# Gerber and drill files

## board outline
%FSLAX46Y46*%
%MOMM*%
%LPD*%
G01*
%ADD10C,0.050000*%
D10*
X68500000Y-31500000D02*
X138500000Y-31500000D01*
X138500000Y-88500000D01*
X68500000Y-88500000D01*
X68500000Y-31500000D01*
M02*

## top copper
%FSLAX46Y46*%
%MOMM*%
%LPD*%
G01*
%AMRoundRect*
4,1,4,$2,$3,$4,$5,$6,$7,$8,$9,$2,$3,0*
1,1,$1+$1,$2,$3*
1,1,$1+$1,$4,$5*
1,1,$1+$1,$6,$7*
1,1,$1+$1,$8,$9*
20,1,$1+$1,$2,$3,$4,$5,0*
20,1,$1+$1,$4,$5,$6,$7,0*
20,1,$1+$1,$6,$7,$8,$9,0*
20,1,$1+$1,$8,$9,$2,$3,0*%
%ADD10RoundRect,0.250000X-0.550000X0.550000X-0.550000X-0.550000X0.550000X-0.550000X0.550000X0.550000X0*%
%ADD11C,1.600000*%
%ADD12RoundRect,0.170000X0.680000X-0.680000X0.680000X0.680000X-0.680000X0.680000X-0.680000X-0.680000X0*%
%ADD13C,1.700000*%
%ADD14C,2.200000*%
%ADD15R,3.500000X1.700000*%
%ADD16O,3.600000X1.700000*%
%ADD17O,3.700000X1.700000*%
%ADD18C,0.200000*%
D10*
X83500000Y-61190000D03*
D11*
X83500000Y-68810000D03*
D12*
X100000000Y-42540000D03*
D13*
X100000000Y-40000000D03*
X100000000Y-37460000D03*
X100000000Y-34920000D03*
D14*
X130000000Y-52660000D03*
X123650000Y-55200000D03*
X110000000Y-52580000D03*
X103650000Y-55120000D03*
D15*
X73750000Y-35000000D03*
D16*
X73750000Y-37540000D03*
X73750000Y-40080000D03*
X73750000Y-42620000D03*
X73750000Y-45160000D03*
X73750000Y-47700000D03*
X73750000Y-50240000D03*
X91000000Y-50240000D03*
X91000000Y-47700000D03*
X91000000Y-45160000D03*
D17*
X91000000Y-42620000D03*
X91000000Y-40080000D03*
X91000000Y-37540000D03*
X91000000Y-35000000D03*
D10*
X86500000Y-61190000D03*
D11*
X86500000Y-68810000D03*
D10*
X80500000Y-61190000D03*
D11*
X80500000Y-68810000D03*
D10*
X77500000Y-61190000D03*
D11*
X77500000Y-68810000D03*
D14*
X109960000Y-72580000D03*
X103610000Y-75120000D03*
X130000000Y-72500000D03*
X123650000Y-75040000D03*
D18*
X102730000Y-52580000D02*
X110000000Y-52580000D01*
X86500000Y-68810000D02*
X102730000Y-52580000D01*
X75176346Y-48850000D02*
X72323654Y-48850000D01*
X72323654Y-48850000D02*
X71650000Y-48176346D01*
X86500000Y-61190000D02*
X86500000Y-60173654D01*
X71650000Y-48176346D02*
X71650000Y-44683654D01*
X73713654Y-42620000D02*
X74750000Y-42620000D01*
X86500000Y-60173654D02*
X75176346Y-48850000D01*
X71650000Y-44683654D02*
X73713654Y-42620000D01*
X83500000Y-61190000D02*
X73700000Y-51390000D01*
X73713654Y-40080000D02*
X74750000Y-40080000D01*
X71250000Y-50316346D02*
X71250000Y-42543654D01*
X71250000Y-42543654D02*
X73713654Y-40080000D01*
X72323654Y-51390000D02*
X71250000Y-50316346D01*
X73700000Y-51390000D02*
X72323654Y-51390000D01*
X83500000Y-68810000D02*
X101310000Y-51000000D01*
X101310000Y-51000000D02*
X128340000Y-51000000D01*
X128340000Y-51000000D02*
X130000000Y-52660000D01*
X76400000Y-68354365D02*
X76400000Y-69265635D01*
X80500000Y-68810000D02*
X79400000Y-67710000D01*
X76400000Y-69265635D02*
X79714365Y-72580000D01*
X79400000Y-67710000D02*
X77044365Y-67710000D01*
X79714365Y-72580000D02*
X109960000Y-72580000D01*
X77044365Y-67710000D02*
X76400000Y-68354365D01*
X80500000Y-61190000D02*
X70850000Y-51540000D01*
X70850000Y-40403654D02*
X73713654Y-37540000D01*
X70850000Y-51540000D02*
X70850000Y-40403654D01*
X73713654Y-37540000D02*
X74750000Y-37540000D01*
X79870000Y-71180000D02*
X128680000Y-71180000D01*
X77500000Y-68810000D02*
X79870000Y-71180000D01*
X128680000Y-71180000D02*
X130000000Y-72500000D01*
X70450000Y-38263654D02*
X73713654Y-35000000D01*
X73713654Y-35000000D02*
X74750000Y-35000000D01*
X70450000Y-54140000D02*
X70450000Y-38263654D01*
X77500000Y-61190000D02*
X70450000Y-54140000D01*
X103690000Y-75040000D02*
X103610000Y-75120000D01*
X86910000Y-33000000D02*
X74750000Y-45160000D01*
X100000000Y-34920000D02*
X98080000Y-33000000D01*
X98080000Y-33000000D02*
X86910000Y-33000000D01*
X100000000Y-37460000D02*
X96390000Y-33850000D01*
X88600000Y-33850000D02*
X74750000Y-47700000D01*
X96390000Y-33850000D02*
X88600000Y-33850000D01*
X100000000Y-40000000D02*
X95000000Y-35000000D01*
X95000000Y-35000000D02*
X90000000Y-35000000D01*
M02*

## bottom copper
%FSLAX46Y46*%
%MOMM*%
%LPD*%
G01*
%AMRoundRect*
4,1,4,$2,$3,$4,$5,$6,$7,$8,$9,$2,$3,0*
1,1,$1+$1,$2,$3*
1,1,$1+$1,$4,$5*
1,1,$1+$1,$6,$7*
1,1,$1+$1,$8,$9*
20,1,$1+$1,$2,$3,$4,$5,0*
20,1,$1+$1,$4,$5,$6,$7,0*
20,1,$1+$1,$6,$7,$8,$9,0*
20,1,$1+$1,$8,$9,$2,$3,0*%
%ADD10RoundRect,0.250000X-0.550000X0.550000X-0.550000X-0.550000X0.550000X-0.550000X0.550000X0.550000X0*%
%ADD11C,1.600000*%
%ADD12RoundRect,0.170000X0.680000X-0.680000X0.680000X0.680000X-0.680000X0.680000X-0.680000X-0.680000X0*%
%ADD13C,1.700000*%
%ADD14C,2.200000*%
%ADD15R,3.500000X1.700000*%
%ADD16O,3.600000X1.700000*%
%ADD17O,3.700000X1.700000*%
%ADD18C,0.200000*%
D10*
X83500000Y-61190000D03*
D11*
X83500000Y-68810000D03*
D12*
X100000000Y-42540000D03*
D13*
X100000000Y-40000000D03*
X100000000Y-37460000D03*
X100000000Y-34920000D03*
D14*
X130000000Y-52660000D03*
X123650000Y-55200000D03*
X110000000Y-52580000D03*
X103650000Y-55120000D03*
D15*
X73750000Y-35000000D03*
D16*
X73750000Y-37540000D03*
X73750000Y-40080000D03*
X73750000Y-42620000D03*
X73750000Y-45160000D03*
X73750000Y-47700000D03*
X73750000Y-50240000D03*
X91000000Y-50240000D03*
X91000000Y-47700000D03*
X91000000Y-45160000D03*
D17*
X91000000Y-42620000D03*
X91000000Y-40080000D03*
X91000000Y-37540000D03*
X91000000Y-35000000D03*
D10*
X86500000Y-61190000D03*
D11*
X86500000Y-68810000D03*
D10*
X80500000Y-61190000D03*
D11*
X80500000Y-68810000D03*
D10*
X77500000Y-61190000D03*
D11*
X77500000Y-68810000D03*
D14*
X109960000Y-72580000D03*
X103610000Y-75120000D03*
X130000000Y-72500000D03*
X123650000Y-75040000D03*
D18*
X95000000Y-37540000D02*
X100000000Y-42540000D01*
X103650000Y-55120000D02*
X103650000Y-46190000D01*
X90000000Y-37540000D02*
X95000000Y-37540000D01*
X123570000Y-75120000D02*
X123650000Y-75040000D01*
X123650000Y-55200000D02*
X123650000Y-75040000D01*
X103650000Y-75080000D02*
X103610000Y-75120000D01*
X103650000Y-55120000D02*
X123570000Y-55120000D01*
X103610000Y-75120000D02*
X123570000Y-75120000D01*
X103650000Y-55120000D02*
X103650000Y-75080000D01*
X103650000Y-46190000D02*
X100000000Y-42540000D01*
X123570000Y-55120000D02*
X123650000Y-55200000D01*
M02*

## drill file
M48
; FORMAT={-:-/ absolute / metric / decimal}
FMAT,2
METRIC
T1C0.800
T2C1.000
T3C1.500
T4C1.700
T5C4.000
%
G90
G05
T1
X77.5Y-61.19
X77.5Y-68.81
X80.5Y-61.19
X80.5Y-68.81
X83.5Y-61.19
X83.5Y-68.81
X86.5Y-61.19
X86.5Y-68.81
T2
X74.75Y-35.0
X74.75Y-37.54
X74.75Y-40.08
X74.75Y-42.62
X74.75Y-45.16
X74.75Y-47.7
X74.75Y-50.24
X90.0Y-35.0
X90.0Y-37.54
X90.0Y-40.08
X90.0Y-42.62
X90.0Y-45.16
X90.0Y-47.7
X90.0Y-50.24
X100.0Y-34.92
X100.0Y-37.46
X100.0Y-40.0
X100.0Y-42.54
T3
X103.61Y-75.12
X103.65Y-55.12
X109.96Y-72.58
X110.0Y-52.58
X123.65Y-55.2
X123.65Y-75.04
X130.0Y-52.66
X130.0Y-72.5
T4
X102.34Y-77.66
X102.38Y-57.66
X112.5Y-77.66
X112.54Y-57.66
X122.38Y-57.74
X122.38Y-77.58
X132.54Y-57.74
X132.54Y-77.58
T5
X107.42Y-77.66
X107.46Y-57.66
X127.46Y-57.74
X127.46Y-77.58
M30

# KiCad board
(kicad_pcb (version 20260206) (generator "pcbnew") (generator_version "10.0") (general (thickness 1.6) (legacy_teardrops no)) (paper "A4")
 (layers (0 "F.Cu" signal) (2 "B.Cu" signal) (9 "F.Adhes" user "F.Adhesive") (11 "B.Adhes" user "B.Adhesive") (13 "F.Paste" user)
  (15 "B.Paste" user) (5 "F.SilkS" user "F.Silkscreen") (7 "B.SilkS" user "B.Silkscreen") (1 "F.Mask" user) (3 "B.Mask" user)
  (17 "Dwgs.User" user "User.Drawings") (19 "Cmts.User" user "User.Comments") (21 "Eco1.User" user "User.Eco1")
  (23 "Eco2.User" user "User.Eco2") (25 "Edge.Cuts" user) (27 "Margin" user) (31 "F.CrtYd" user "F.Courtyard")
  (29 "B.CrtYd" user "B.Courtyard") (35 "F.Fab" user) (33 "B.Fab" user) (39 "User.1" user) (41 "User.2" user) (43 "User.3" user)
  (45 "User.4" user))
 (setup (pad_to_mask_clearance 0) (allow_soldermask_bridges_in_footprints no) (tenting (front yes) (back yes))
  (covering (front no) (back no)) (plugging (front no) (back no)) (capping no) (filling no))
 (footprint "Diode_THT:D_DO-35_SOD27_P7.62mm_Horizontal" (layer "F.Cu") (at 83.5 61.19 -90)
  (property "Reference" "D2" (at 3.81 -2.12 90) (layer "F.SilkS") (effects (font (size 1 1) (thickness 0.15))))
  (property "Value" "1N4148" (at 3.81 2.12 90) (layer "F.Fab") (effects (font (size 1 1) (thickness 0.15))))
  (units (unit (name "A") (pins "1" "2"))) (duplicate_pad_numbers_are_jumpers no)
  (pad "1" thru_hole roundrect (at 0 0 270) (size 1.6 1.6) (drill 0.8) (layers "*.Cu" "*.Mask") (remove_unused_layers no)
   (roundrect_rratio 0.15625) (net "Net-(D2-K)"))
  (pad "2" thru_hole circle (at 7.62 0 270) (size 1.6 1.6) (drill 0.8) (layers "*.Cu" "*.Mask") (remove_unused_layers no) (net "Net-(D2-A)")))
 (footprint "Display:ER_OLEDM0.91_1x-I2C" (layer "F.Cu") (at 100 42.54 90)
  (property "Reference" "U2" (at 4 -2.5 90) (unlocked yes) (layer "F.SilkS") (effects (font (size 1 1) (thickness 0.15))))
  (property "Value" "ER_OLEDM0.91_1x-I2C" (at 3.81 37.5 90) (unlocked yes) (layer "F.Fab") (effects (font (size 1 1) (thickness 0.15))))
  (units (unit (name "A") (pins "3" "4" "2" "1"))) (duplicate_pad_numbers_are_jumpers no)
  (pad "1" thru_hole roundrect (at 0 0 90) (size 1.7 1.7) (drill 1) (layers "*.Cu" "*.Mask") (remove_unused_layers no)
   (roundrect_rratio 0.1) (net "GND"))
  (pad "2" thru_hole circle (at 2.54 0 90) (size 1.7 1.7) (drill 1) (layers "*.Cu" "*.Mask") (remove_unused_layers no) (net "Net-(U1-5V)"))
  (pad "3" thru_hole circle (at 5.08 0 90) (size 1.7 1.7) (drill 1) (layers "*.Cu" "*.Mask") (remove_unused_layers no)
   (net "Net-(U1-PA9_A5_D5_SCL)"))
  (pad "4" thru_hole circle (at 7.62 0 90) (size 1.7 1.7) (drill 1) (layers "*.Cu" "*.Mask") (remove_unused_layers no)
   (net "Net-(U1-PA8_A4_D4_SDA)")))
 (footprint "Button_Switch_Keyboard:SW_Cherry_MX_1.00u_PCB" (layer "F.Cu") (at 130 52.66)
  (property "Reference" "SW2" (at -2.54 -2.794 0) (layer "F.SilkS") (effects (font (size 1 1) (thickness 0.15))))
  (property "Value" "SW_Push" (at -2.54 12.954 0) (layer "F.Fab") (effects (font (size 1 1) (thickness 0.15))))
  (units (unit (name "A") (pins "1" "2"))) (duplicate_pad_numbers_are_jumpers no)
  (pad "" np_thru_hole circle (at -7.62 5.08) (size 1.7 1.7) (drill 1.7) (layers "*.Cu" "*.Mask"))
  (pad "" np_thru_hole circle (at -2.54 5.08) (size 4 4) (drill 4) (layers "*.Cu" "*.Mask"))
  (pad "" np_thru_hole circle (at 2.54 5.08) (size 1.7 1.7) (drill 1.7) (layers "*.Cu" "*.Mask"))
  (pad "1" thru_hole circle (at 0 0) (size 2.2 2.2) (drill 1.5) (layers "*.Cu" "*.Mask") (remove_unused_layers no) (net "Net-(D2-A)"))
  (pad "2" thru_hole circle (at -6.35 2.54) (size 2.2 2.2) (drill 1.5) (layers "*.Cu" "*.Mask") (remove_unused_layers no) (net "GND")))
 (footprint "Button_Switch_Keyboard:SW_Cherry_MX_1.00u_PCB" (layer "F.Cu") (at 110 52.58)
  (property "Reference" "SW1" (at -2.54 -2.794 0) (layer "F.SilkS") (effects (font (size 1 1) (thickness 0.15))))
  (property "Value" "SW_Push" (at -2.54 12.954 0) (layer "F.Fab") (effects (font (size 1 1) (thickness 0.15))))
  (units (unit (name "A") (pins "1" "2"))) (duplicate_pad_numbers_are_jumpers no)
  (pad "" np_thru_hole circle (at -7.62 5.08) (size 1.7 1.7) (drill 1.7) (layers "*.Cu" "*.Mask"))
  (pad "" np_thru_hole circle (at -2.54 5.08) (size 4 4) (drill 4) (layers "*.Cu" "*.Mask"))
  (pad "" np_thru_hole circle (at 2.54 5.08) (size 1.7 1.7) (drill 1.7) (layers "*.Cu" "*.Mask"))
  (pad "1" thru_hole circle (at 0 0) (size 2.2 2.2) (drill 1.5) (layers "*.Cu" "*.Mask") (remove_unused_layers no) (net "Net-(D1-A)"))
  (pad "2" thru_hole circle (at -6.35 2.54) (size 2.2 2.2) (drill 1.5) (layers "*.Cu" "*.Mask") (remove_unused_layers no) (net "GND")))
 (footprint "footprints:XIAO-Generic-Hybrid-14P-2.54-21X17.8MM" (layer "F.Cu") (at 82.375 42.62)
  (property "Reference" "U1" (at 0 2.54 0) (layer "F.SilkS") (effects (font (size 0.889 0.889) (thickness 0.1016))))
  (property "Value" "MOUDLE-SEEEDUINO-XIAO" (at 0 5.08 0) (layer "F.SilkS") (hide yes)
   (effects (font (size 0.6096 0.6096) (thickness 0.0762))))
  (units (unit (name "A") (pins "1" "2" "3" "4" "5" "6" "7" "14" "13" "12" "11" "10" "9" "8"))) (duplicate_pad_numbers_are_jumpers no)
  (pad "1" thru_hole rect (at -7.625 -7.62) (size 3.5 1.7) (drill 1 (offset -1 0)) (layers "*.Cu" "*.Mask") (remove_unused_layers no)
   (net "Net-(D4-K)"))
  (pad "2" thru_hole oval (at -7.625 -5.08) (size 3.6 1.7) (drill 1 (offset -1 0)) (layers "*.Cu" "*.Mask") (remove_unused_layers no)
   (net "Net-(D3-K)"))
  (pad "3" thru_hole oval (at -7.625 -2.54) (size 3.6 1.7) (drill 1 (offset -1 0)) (layers "*.Cu" "*.Mask") (remove_unused_layers no)
   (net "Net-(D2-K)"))
  (pad "4" thru_hole oval (at -7.625 0) (size 3.6 1.7) (drill 1 (offset -1 0)) (layers "*.Cu" "*.Mask") (remove_unused_layers no)
   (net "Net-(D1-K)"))
  (pad "5" thru_hole oval (at -7.625 2.54) (size 3.6 1.7) (drill 1 (offset -1 0)) (layers "*.Cu" "*.Mask") (remove_unused_layers no)
   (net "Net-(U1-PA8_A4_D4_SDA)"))
  (pad "6" thru_hole oval (at -7.625 5.08 180) (size 3.6 1.7) (drill 1 (offset 1 0)) (layers "*.Cu" "*.Mask") (remove_unused_layers no)
   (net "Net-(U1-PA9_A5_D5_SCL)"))
  (pad "7" thru_hole oval (at -7.625 7.62) (size 3.6 1.7) (drill 1 (offset -1 0)) (layers "*.Cu" "*.Mask") (remove_unused_layers no)
   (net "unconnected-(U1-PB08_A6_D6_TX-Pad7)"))
  (pad "8" thru_hole oval (at 7.625 7.62) (size 3.6 1.7) (drill 1 (offset 1 0)) (layers "*.Cu" "*.Mask") (remove_unused_layers no)
   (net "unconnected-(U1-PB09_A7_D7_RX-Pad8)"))
  (pad "9" thru_hole oval (at 7.625 5.08) (size 3.6 1.7) (drill 1 (offset 1 0)) (layers "*.Cu" "*.Mask") (remove_unused_layers no)
   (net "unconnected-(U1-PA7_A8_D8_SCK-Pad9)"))
  (pad "10" thru_hole oval (at 7.625 2.54) (size 3.6 1.7) (drill 1 (offset 1 0)) (layers "*.Cu" "*.Mask") (remove_unused_layers no)
   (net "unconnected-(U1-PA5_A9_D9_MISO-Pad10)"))
  (pad "11" thru_hole oval (at 7.625 0) (size 3.7 1.7) (drill 1 (offset 1 0)) (layers "*.Cu" "*.Mask") (remove_unused_layers no)
   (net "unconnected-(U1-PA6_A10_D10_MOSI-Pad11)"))
  (pad "12" thru_hole oval (at 7.625 -2.54) (size 3.7 1.7) (drill 1 (offset 1 0)) (layers "*.Cu" "*.Mask") (remove_unused_layers no)
   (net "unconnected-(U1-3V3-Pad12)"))
  (pad "13" thru_hole oval (at 7.625 -5.08) (size 3.7 1.7) (drill 1 (offset 1 0)) (layers "*.Cu" "*.Mask") (remove_unused_layers no)
   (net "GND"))
  (pad "14" thru_hole oval (at 7.625 -7.62) (size 3.7 1.7) (drill 1 (offset 1 0)) (layers "*.Cu" "*.Mask") (remove_unused_layers no)
   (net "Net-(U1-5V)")))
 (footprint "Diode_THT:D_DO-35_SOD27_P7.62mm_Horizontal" (layer "F.Cu") (at 86.5 61.19 -90)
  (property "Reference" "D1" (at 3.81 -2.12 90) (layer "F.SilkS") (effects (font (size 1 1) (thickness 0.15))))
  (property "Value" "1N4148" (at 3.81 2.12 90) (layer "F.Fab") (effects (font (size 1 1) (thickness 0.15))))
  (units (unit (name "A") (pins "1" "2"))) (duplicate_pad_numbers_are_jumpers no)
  (pad "1" thru_hole roundrect (at 0 0 270) (size 1.6 1.6) (drill 0.8) (layers "*.Cu" "*.Mask") (remove_unused_layers no)
   (roundrect_rratio 0.15625) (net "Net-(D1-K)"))
  (pad "2" thru_hole circle (at 7.62 0 270) (size 1.6 1.6) (drill 0.8) (layers "*.Cu" "*.Mask") (remove_unused_layers no) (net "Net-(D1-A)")))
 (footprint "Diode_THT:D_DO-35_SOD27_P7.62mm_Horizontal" (layer "F.Cu") (at 80.5 61.19 -90)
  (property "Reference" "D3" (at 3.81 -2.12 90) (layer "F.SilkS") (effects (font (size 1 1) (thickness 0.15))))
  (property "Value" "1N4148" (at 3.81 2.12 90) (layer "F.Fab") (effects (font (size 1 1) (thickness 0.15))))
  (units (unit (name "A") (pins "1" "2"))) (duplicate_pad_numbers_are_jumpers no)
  (pad "1" thru_hole roundrect (at 0 0 270) (size 1.6 1.6) (drill 0.8) (layers "*.Cu" "*.Mask") (remove_unused_layers no)
   (roundrect_rratio 0.15625) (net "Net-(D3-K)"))
  (pad "2" thru_hole circle (at 7.62 0 270) (size 1.6 1.6) (drill 0.8) (layers "*.Cu" "*.Mask") (remove_unused_layers no) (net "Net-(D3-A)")))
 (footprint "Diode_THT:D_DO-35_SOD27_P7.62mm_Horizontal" (layer "F.Cu") (at 77.5 61.19 -90)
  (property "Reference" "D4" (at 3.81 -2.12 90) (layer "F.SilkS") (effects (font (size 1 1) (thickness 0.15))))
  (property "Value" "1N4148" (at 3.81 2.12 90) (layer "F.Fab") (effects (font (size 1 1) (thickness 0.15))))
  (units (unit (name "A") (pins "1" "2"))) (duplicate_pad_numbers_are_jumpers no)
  (pad "1" thru_hole roundrect (at 0 0 270) (size 1.6 1.6) (drill 0.8) (layers "*.Cu" "*.Mask") (remove_unused_layers no)
   (roundrect_rratio 0.15625) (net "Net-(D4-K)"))
  (pad "2" thru_hole circle (at 7.62 0 270) (size 1.6 1.6) (drill 0.8) (layers "*.Cu" "*.Mask") (remove_unused_layers no) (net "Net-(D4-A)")))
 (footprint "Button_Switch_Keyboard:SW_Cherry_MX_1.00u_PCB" (layer "F.Cu") (at 109.96 72.58)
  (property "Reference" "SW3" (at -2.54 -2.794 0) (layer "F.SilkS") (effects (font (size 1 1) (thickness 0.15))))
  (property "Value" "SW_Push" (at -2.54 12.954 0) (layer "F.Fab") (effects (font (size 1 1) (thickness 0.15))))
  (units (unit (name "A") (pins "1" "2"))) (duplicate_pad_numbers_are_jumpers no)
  (pad "" np_thru_hole circle (at -7.62 5.08) (size 1.7 1.7) (drill 1.7) (layers "*.Cu" "*.Mask"))
  (pad "" np_thru_hole circle (at -2.54 5.08) (size 4 4) (drill 4) (layers "*.Cu" "*.Mask"))
  (pad "" np_thru_hole circle (at 2.54 5.08) (size 1.7 1.7) (drill 1.7) (layers "*.Cu" "*.Mask"))
  (pad "1" thru_hole circle (at 0 0) (size 2.2 2.2) (drill 1.5) (layers "*.Cu" "*.Mask") (remove_unused_layers no) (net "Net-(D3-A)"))
  (pad "2" thru_hole circle (at -6.35 2.54) (size 2.2 2.2) (drill 1.5) (layers "*.Cu" "*.Mask") (remove_unused_layers no) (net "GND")))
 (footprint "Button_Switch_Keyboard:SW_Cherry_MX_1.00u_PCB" (layer "F.Cu") (at 130 72.5)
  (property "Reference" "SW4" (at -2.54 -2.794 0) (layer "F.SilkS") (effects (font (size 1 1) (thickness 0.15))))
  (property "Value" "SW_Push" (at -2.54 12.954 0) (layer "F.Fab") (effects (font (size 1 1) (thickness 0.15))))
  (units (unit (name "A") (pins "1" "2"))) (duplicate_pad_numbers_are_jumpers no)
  (pad "" np_thru_hole circle (at -7.62 5.08) (size 1.7 1.7) (drill 1.7) (layers "*.Cu" "*.Mask"))
  (pad "" np_thru_hole circle (at -2.54 5.08) (size 4 4) (drill 4) (layers "*.Cu" "*.Mask"))
  (pad "" np_thru_hole circle (at 2.54 5.08) (size 1.7 1.7) (drill 1.7) (layers "*.Cu" "*.Mask"))
  (pad "1" thru_hole circle (at 0 0) (size 2.2 2.2) (drill 1.5) (layers "*.Cu" "*.Mask") (remove_unused_layers no) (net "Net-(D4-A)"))
  (pad "2" thru_hole circle (at -6.35 2.54) (size 2.2 2.2) (drill 1.5) (layers "*.Cu" "*.Mask") (remove_unused_layers no) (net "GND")))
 (gr_rect (start 68.5 31.5) (end 138.5 88.5) (stroke (width 0.05) (type default)) (fill no) (layer "Edge.Cuts"))
 (segment (start 102.73 52.58) (end 110 52.58) (width 0.2) (layer "F.Cu") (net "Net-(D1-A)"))
 (segment (start 86.5 68.81) (end 102.73 52.58) (width 0.2) (layer "F.Cu") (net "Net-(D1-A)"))
 (segment (start 75.176346 48.85) (end 72.323654 48.85) (width 0.2) (layer "F.Cu") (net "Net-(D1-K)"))
 (segment (start 72.323654 48.85) (end 71.65 48.176346) (width 0.2) (layer "F.Cu") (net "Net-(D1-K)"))
 (segment (start 86.5 61.19) (end 86.5 60.173654) (width 0.2) (layer "F.Cu") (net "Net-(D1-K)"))
 (segment (start 71.65 48.176346) (end 71.65 44.683654) (width 0.2) (layer "F.Cu") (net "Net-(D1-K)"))
 (segment (start 73.713654 42.62) (end 74.75 42.62) (width 0.2) (layer "F.Cu") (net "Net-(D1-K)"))
 (segment (start 86.5 60.173654) (end 75.176346 48.85) (width 0.2) (layer "F.Cu") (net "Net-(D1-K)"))
 (segment (start 71.65 44.683654) (end 73.713654 42.62) (width 0.2) (layer "F.Cu") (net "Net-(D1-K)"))
 (segment (start 83.5 61.19) (end 73.7 51.39) (width 0.2) (layer "F.Cu") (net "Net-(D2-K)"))
 (segment (start 73.713654 40.08) (end 74.75 40.08) (width 0.2) (layer "F.Cu") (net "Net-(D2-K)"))
 (segment (start 71.25 50.316346) (end 71.25 42.543654) (width 0.2) (layer "F.Cu") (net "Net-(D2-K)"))
 (segment (start 71.25 42.543654) (end 73.713654 40.08) (width 0.2) (layer "F.Cu") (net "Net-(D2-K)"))
 (segment (start 72.323654 51.39) (end 71.25 50.316346) (width 0.2) (layer "F.Cu") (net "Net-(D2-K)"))
 (segment (start 73.7 51.39) (end 72.323654 51.39) (width 0.2) (layer "F.Cu") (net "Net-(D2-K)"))
 (segment (start 83.5 68.81) (end 101.31 51) (width 0.2) (layer "F.Cu") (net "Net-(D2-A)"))
 (segment (start 101.31 51) (end 128.34 51) (width 0.2) (layer "F.Cu") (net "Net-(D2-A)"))
 (segment (start 128.34 51) (end 130 52.66) (width 0.2) (layer "F.Cu") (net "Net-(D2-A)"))
 (segment (start 76.4 68.354365) (end 76.4 69.265635) (width 0.2) (layer "F.Cu") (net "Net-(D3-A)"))
 (segment (start 80.5 68.81) (end 79.4 67.71) (width 0.2) (layer "F.Cu") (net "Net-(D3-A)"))
 (segment (start 76.4 69.265635) (end 79.714365 72.58) (width 0.2) (layer "F.Cu") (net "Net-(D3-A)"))
 (segment (start 79.4 67.71) (end 77.044365 67.71) (width 0.2) (layer "F.Cu") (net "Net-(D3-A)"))
 (segment (start 79.714365 72.58) (end 109.96 72.58) (width 0.2) (layer "F.Cu") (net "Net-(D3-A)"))
 (segment (start 77.044365 67.71) (end 76.4 68.354365) (width 0.2) (layer "F.Cu") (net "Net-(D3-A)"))
 (segment (start 80.5 61.19) (end 70.85 51.54) (width 0.2) (layer "F.Cu") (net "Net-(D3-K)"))
 (segment (start 70.85 40.403654) (end 73.713654 37.54) (width 0.2) (layer "F.Cu") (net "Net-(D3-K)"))
 (segment (start 70.85 51.54) (end 70.85 40.403654) (width 0.2) (layer "F.Cu") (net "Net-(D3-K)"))
 (segment (start 73.713654 37.54) (end 74.75 37.54) (width 0.2) (layer "F.Cu") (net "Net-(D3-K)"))
 (segment (start 79.87 71.18) (end 128.68 71.18) (width 0.2) (layer "F.Cu") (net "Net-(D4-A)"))
 (segment (start 77.5 68.81) (end 79.87 71.18) (width 0.2) (layer "F.Cu") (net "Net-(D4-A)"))
 (segment (start 128.68 71.18) (end 130 72.5) (width 0.2) (layer "F.Cu") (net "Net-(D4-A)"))
 (segment (start 70.45 38.263654) (end 73.713654 35) (width 0.2) (layer "F.Cu") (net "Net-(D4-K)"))
 (segment (start 73.713654 35) (end 74.75 35) (width 0.2) (layer "F.Cu") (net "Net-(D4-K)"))
 (segment (start 70.45 54.14) (end 70.45 38.263654) (width 0.2) (layer "F.Cu") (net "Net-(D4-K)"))
 (segment (start 77.5 61.19) (end 70.45 54.14) (width 0.2) (layer "F.Cu") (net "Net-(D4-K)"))
 (segment (start 103.69 75.04) (end 103.61 75.12) (width 0.2) (layer "F.Cu") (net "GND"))
 (segment (start 95 37.54) (end 100 42.54) (width 0.2) (layer "B.Cu") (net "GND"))
 (segment (start 103.65 55.12) (end 103.65 46.19) (width 0.2) (layer "B.Cu") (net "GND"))
 (segment (start 90 37.54) (end 95 37.54) (width 0.2) (layer "B.Cu") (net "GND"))
 (segment (start 123.57 75.12) (end 123.65 75.04) (width 0.2) (layer "B.Cu") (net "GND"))
 (segment (start 123.65 55.2) (end 123.65 75.04) (width 0.2) (layer "B.Cu") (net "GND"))
 (segment (start 103.65 75.08) (end 103.61 75.12) (width 0.2) (layer "B.Cu") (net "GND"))
 (segment (start 103.65 55.12) (end 123.57 55.12) (width 0.2) (layer "B.Cu") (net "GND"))
 (segment (start 103.61 75.12) (end 123.57 75.12) (width 0.2) (layer "B.Cu") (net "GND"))
 (segment (start 103.65 55.12) (end 103.65 75.08) (width 0.2) (layer "B.Cu") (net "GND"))
 (segment (start 103.65 46.19) (end 100 42.54) (width 0.2) (layer "B.Cu") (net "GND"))
 (segment (start 123.57 55.12) (end 123.65 55.2) (width 0.2) (layer "B.Cu") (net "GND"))
 (segment (start 86.91 33) (end 74.75 45.16) (width 0.2) (layer "F.Cu") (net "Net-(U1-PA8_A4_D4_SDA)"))
 (segment (start 100 34.92) (end 98.08 33) (width 0.2) (layer "F.Cu") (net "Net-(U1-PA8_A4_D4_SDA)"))
 (segment (start 98.08 33) (end 86.91 33) (width 0.2) (layer "F.Cu") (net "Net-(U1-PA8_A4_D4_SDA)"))
 (segment (start 100 37.46) (end 96.39 33.85) (width 0.2) (layer "F.Cu") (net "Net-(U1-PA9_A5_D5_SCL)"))
 (segment (start 88.6 33.85) (end 74.75 47.7) (width 0.2) (layer "F.Cu") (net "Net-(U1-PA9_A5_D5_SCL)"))
 (segment (start 96.39 33.85) (end 88.6 33.85) (width 0.2) (layer "F.Cu") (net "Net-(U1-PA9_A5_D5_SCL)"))
 (segment (start 100 40) (end 95 35) (width 0.2) (layer "F.Cu") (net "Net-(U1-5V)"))
 (segment (start 95 35) (end 90 35) (width 0.2) (layer "F.Cu") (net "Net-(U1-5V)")))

